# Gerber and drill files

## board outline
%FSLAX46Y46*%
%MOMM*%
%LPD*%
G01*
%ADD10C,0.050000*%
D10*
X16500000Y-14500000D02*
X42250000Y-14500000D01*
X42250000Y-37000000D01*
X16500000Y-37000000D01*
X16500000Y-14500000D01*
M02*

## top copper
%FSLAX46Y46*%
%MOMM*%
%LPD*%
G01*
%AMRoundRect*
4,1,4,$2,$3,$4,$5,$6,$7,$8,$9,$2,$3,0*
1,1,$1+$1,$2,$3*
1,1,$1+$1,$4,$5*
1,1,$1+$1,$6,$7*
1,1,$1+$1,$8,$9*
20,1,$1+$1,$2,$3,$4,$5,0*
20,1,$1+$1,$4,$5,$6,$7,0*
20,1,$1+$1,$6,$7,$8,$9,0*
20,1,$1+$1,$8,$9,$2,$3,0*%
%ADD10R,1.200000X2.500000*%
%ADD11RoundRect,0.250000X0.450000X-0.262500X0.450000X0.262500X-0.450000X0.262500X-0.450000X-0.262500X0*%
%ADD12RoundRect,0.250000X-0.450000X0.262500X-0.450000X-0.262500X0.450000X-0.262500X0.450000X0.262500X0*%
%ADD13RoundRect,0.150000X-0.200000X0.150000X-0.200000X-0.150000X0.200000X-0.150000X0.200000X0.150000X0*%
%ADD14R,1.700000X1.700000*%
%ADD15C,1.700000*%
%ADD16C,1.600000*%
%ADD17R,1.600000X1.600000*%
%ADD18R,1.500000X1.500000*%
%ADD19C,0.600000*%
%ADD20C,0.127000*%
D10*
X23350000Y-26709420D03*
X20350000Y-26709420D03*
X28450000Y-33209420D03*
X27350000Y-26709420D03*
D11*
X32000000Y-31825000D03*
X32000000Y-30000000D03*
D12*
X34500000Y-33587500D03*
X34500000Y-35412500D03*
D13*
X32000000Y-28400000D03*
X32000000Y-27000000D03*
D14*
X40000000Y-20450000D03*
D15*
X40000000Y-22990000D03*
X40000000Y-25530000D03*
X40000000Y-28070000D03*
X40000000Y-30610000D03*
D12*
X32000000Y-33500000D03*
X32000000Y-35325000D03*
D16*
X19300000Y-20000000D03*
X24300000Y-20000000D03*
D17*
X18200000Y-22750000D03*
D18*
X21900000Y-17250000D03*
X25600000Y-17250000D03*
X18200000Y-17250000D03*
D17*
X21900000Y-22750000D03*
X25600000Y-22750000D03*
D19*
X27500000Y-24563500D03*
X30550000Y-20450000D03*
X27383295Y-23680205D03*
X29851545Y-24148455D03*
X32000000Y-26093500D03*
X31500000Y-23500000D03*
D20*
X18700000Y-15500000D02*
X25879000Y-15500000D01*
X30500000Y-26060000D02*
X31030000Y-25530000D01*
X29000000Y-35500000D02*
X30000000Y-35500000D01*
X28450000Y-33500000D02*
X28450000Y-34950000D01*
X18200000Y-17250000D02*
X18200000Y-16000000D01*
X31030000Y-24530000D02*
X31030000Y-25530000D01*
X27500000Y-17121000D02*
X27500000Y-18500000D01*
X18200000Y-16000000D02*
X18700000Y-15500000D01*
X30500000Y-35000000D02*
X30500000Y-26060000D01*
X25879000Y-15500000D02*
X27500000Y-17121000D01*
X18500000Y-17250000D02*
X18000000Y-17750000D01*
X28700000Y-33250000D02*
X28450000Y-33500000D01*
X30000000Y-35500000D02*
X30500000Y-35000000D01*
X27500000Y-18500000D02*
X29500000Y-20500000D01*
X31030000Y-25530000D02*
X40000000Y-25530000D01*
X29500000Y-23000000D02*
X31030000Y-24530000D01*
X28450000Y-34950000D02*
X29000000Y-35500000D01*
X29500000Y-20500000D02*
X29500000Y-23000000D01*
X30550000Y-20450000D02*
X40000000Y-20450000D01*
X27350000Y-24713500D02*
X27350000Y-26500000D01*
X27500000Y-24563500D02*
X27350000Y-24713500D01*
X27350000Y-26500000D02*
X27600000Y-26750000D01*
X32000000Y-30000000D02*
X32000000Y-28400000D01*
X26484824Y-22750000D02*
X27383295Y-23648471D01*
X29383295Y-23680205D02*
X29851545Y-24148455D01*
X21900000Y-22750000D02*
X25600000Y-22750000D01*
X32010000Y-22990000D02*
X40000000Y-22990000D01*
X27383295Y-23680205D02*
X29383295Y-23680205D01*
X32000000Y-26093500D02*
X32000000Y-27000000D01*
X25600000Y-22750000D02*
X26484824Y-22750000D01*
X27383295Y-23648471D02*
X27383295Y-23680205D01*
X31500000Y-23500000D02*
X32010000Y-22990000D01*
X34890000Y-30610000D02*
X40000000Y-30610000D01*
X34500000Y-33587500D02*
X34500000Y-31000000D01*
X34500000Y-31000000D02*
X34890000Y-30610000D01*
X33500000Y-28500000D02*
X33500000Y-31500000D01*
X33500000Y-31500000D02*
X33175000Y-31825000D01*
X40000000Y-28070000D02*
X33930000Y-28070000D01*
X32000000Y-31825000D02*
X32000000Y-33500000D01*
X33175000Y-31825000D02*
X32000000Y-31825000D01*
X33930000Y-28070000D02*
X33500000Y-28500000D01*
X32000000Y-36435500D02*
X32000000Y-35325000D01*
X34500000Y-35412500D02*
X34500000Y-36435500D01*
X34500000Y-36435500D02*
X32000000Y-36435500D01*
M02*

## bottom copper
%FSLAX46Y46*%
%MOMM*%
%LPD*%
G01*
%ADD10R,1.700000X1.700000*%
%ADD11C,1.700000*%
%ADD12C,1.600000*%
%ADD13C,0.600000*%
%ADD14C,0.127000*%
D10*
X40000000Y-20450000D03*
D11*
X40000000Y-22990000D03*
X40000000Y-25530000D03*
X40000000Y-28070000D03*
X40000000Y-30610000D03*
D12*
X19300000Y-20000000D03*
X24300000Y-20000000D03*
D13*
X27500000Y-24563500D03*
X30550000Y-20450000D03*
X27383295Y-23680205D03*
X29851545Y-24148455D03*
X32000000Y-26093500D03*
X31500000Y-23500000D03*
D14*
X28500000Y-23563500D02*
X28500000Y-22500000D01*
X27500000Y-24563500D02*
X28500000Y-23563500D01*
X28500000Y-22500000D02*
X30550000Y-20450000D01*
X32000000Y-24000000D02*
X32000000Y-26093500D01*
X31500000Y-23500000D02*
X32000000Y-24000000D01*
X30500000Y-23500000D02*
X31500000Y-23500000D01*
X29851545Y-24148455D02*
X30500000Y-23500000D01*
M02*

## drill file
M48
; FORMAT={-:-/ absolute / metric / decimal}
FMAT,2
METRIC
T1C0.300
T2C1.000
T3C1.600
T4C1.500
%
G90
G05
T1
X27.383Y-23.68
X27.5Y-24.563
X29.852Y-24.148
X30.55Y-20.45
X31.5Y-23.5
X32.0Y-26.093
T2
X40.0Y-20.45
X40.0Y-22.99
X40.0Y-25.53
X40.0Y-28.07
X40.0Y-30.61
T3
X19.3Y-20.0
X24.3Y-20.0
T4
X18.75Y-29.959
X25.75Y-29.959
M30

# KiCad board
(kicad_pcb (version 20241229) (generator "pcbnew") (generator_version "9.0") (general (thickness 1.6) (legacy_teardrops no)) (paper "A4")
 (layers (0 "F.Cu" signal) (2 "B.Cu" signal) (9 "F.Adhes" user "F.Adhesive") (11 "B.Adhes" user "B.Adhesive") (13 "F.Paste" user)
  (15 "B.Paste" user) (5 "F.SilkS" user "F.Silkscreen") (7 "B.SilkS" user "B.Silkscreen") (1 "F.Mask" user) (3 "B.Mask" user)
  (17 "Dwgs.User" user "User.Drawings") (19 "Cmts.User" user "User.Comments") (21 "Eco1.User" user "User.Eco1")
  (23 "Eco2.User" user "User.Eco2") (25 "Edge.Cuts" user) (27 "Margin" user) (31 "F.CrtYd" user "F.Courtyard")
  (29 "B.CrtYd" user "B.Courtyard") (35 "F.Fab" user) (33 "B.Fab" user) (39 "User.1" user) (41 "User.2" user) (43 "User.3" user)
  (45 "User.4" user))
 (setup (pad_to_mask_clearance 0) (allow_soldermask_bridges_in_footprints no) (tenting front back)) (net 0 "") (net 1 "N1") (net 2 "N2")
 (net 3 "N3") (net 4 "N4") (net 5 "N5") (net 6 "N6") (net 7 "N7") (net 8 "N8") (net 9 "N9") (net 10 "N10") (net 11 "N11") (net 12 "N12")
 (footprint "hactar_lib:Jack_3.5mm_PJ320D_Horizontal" (layer "F.Cu") (at 23.35 29.95942)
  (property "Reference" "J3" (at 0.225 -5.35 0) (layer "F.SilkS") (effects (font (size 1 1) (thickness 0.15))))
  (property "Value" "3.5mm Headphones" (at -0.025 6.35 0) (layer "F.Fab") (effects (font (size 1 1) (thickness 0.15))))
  (pad "" np_thru_hole circle (at -4.6 0) (size 1.5 1.5) (drill 1.5) (layers "*.Cu" "*.Mask"))
  (pad "" np_thru_hole circle (at 2.4 0) (size 1.5 1.5) (drill 1.5) (layers "*.Cu" "*.Mask"))
  (pad "R1" smd rect (at 0 -3.25) (size 1.2 2.5) (layers "F.Cu" "F.Mask" "F.Paste") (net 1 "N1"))
  (pad "R2" smd rect (at -3 -3.25) (size 1.2 2.5) (layers "F.Cu" "F.Mask" "F.Paste") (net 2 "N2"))
  (pad "S" smd rect (at 5.1 3.25) (size 1.2 2.5) (layers "F.Cu" "F.Mask" "F.Paste") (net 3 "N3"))
  (pad "T" smd rect (at 4 -3.25) (size 1.2 2.5) (layers "F.Cu" "F.Mask" "F.Paste") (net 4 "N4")))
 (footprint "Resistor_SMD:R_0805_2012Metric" (layer "F.Cu") (at 32 30.9125 90)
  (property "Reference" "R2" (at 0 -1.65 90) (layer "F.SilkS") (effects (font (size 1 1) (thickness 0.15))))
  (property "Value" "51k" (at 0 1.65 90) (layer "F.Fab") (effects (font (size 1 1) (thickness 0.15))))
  (pad "1" smd roundrect (at -0.9125 0 90) (size 1.025 1.4) (layers "F.Cu" "F.Mask" "F.Paste") (roundrect_rratio 0.243902) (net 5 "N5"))
  (pad "2" smd roundrect (at 0.9125 0 90) (size 1.025 1.4) (layers "F.Cu" "F.Mask" "F.Paste") (roundrect_rratio 0.243902) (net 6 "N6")))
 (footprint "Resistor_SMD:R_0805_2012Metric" (layer "F.Cu") (at 34.5 34.5 -90)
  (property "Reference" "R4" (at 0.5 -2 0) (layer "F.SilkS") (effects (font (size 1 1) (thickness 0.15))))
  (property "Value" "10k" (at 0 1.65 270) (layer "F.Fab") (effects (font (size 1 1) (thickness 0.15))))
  (pad "1" smd roundrect (at -0.9125 0 270) (size 1.025 1.4) (layers "F.Cu" "F.Mask" "F.Paste") (roundrect_rratio 0.243902) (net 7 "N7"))
  (pad "2" smd roundrect (at 0.9125 0 270) (size 1.025 1.4) (layers "F.Cu" "F.Mask" "F.Paste") (roundrect_rratio 0.243902) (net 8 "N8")))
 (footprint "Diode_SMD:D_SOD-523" (layer "F.Cu") (at 32 27.7 90)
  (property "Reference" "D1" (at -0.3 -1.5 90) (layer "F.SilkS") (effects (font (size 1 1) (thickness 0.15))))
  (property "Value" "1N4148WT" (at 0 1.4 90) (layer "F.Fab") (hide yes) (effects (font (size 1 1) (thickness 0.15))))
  (pad "1" smd roundrect (at -0.7 0 270) (size 0.6 0.7) (layers "F.Cu" "F.Mask" "F.Paste") (roundrect_rratio 0.25) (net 6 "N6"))
  (pad "2" smd roundrect (at 0.7 0 270) (size 0.6 0.7) (layers "F.Cu" "F.Mask" "F.Paste") (roundrect_rratio 0.25) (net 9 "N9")))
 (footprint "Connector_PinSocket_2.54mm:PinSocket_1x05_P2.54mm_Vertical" (layer "F.Cu") (at 40 20.45)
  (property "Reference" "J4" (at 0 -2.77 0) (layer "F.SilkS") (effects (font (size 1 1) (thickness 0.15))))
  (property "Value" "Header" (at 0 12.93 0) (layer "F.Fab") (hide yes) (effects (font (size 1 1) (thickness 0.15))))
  (pad "1" thru_hole rect (at 0 0) (size 1.7 1.7) (drill 1) (layers "*.Cu" "*.Mask") (remove_unused_layers no) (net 4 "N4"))
  (pad "2" thru_hole circle (at 0 2.54) (size 1.7 1.7) (drill 1) (layers "*.Cu" "*.Mask") (remove_unused_layers no) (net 9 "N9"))
  (pad "3" thru_hole circle (at 0 5.08) (size 1.7 1.7) (drill 1) (layers "*.Cu" "*.Mask") (remove_unused_layers no) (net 3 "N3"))
  (pad "4" thru_hole circle (at 0 7.62) (size 1.7 1.7) (drill 1) (layers "*.Cu" "*.Mask") (remove_unused_layers no) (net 5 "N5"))
  (pad "5" thru_hole circle (at 0 10.16) (size 1.7 1.7) (drill 1) (layers "*.Cu" "*.Mask") (remove_unused_layers no) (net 7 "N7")))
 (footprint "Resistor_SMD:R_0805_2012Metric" (layer "F.Cu") (at 32 34.4125 -90)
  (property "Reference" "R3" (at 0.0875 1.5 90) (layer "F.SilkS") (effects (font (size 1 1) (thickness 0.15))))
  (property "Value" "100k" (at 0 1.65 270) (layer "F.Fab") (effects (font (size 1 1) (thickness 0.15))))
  (pad "1" smd roundrect (at -0.9125 0 270) (size 1.025 1.4) (layers "F.Cu" "F.Mask" "F.Paste") (roundrect_rratio 0.243902) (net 5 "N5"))
  (pad "2" smd roundrect (at 0.9125 0 270) (size 1.025 1.4) (layers "F.Cu" "F.Mask" "F.Paste") (roundrect_rratio 0.243902) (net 8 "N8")))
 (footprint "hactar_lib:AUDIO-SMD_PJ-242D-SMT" (layer "F.Cu") (at 21.9 20)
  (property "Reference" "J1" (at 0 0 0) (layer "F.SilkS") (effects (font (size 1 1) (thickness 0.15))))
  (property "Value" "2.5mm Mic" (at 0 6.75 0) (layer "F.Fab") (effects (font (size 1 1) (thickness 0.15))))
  (pad "" thru_hole circle (at -2.6 0) (size 1.6 1.6) (drill 1.6) (layers "*.Cu" "*.Mask") (remove_unused_layers no))
  (pad "" thru_hole circle (at 2.4 0) (size 1.6 1.6) (drill 1.6) (layers "*.Cu" "*.Mask") (remove_unused_layers no))
  (pad "R1" smd rect (at -3.7 2.75 180) (size 1.6 1.6) (layers "F.Cu" "F.Mask" "F.Paste") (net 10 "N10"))
  (pad "R2" smd rect (at 0 -2.75 180) (size 1.5 1.5) (layers "F.Cu" "F.Mask" "F.Paste") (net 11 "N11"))
  (pad "R2" smd rect (at 3.7 -2.75 180) (size 1.5 1.5) (layers "F.Cu" "F.Mask" "F.Paste") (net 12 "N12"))
  (pad "S" smd rect (at -3.7 -2.75 180) (size 1.5 1.5) (layers "F.Cu" "F.Mask" "F.Paste") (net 3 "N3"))
  (pad "T" smd rect (at 0 2.75 180) (size 1.6 1.6) (layers "F.Cu" "F.Mask" "F.Paste") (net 9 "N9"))
  (pad "T" smd rect (at 3.7 2.75 180) (size 1.6 1.6) (layers "F.Cu" "F.Mask" "F.Paste") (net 9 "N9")))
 (gr_rect (start 16.5 14.5) (end 42.25 37) (stroke (width 0.05) (type solid)) (fill no) (layer "Edge.Cuts"))
 (segment (start 18.7 15.5) (end 25.879 15.5) (width 0.127) (layer "F.Cu") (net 3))
 (segment (start 30.5 26.06) (end 31.03 25.53) (width 0.127) (layer "F.Cu") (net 3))
 (segment (start 29 35.5) (end 30 35.5) (width 0.127) (layer "F.Cu") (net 3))
 (segment (start 28.45 33.5) (end 28.45 34.95) (width 0.127) (layer "F.Cu") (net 3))
 (segment (start 18.2 17.25) (end 18.2 16) (width 0.127) (layer "F.Cu") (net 3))
 (segment (start 31.03 24.53) (end 31.03 25.53) (width 0.127) (layer "F.Cu") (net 3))
 (segment (start 27.5 17.121) (end 27.5 18.5) (width 0.127) (layer "F.Cu") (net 3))
 (segment (start 18.2 16) (end 18.7 15.5) (width 0.127) (layer "F.Cu") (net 3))
 (segment (start 30.5 35) (end 30.5 26.06) (width 0.127) (layer "F.Cu") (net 3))
 (segment (start 25.879 15.5) (end 27.5 17.121) (width 0.127) (layer "F.Cu") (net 3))
 (segment (start 18.5 17.25) (end 18 17.75) (width 0.127) (layer "F.Cu") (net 3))
 (segment (start 28.7 33.25) (end 28.45 33.5) (width 0.127) (layer "F.Cu") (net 3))
 (segment (start 30 35.5) (end 30.5 35) (width 0.127) (layer "F.Cu") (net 3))
 (segment (start 27.5 18.5) (end 29.5 20.5) (width 0.127) (layer "F.Cu") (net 3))
 (segment (start 31.03 25.53) (end 40 25.53) (width 0.127) (layer "F.Cu") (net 3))
 (segment (start 29.5 23) (end 31.03 24.53) (width 0.127) (layer "F.Cu") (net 3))
 (segment (start 28.45 34.95) (end 29 35.5) (width 0.127) (layer "F.Cu") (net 3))
 (segment (start 29.5 20.5) (end 29.5 23) (width 0.127) (layer "F.Cu") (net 3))
 (segment (start 30.55 20.45) (end 40 20.45) (width 0.127) (layer "F.Cu") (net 4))
 (segment (start 27.35 24.7135) (end 27.35 26.5) (width 0.127) (layer "F.Cu") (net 4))
 (segment (start 27.5 24.5635) (end 27.35 24.7135) (width 0.127) (layer "F.Cu") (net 4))
 (segment (start 27.35 26.5) (end 27.6 26.75) (width 0.127) (layer "F.Cu") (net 4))
 (via (at 27.5 24.5635) (size 0.6) (drill 0.3) (layers "F.Cu" "B.Cu") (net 4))
 (via (at 30.55 20.45) (size 0.6) (drill 0.3) (layers "F.Cu" "B.Cu") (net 4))
 (segment (start 28.5 23.5635) (end 28.5 22.5) (width 0.127) (layer "B.Cu") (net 4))
 (segment (start 27.5 24.5635) (end 28.5 23.5635) (width 0.127) (layer "B.Cu") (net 4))
 (segment (start 28.5 22.5) (end 30.55 20.45) (width 0.127) (layer "B.Cu") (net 4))
 (segment (start 32 30) (end 32 28.4) (width 0.127) (layer "F.Cu") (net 6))
 (segment (start 26.484824 22.75) (end 27.383295 23.648471) (width 0.127) (layer "F.Cu") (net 9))
 (segment (start 29.383295 23.680205) (end 29.851545 24.148455) (width 0.127) (layer "F.Cu") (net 9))
 (segment (start 21.9 22.75) (end 25.6 22.75) (width 0.127) (layer "F.Cu") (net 9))
 (segment (start 32.01 22.99) (end 40 22.99) (width 0.127) (layer "F.Cu") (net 9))
 (segment (start 27.383295 23.680205) (end 29.383295 23.680205) (width 0.127) (layer "F.Cu") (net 9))
 (segment (start 32 26.0935) (end 32 27) (width 0.127) (layer "F.Cu") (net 9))
 (segment (start 25.6 22.75) (end 26.484824 22.75) (width 0.127) (layer "F.Cu") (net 9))
 (segment (start 27.383295 23.648471) (end 27.383295 23.680205) (width 0.127) (layer "F.Cu") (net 9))
 (segment (start 31.5 23.5) (end 32.01 22.99) (width 0.127) (layer "F.Cu") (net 9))
 (via (at 27.383295 23.680205) (size 0.6) (drill 0.3) (layers "F.Cu" "B.Cu") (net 9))
 (via (at 29.851545 24.148455) (size 0.6) (drill 0.3) (layers "F.Cu" "B.Cu") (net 9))
 (via (at 32 26.0935) (size 0.6) (drill 0.3) (layers "F.Cu" "B.Cu") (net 9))
 (via (at 31.5 23.5) (size 0.6) (drill 0.3) (layers "F.Cu" "B.Cu") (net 9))
 (segment (start 32 24) (end 32 26.0935) (width 0.127) (layer "B.Cu") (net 9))
 (segment (start 31.5 23.5) (end 32 24) (width 0.127) (layer "B.Cu") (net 9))
 (segment (start 30.5 23.5) (end 31.5 23.5) (width 0.127) (layer "B.Cu") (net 9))
 (segment (start 29.851545 24.148455) (end 30.5 23.5) (width 0.127) (layer "B.Cu") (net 9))
 (segment (start 34.89 30.61) (end 40 30.61) (width 0.127) (layer "F.Cu") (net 7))
 (segment (start 34.5 33.5875) (end 34.5 31) (width 0.127) (layer "F.Cu") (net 7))
 (segment (start 34.5 31) (end 34.89 30.61) (width 0.127) (layer "F.Cu") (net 7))
 (segment (start 33.5 28.5) (end 33.5 31.5) (width 0.127) (layer "F.Cu") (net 5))
 (segment (start 33.5 31.5) (end 33.175 31.825) (width 0.127) (layer "F.Cu") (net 5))
 (segment (start 40 28.07) (end 33.93 28.07) (width 0.127) (layer "F.Cu") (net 5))
 (segment (start 32 31.825) (end 32 33.5) (width 0.127) (layer "F.Cu") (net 5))
 (segment (start 33.175 31.825) (end 32 31.825) (width 0.127) (layer "F.Cu") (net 5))
 (segment (start 33.93 28.07) (end 33.5 28.5) (width 0.127) (layer "F.Cu") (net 5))
 (segment (start 32 36.4355) (end 32 35.325) (width 0.127) (layer "F.Cu") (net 8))
 (segment (start 34.5 35.4125) (end 34.5 36.4355) (width 0.127) (layer "F.Cu") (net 8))
 (segment (start 34.5 36.4355) (end 32 36.4355) (width 0.127) (layer "F.Cu") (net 8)))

